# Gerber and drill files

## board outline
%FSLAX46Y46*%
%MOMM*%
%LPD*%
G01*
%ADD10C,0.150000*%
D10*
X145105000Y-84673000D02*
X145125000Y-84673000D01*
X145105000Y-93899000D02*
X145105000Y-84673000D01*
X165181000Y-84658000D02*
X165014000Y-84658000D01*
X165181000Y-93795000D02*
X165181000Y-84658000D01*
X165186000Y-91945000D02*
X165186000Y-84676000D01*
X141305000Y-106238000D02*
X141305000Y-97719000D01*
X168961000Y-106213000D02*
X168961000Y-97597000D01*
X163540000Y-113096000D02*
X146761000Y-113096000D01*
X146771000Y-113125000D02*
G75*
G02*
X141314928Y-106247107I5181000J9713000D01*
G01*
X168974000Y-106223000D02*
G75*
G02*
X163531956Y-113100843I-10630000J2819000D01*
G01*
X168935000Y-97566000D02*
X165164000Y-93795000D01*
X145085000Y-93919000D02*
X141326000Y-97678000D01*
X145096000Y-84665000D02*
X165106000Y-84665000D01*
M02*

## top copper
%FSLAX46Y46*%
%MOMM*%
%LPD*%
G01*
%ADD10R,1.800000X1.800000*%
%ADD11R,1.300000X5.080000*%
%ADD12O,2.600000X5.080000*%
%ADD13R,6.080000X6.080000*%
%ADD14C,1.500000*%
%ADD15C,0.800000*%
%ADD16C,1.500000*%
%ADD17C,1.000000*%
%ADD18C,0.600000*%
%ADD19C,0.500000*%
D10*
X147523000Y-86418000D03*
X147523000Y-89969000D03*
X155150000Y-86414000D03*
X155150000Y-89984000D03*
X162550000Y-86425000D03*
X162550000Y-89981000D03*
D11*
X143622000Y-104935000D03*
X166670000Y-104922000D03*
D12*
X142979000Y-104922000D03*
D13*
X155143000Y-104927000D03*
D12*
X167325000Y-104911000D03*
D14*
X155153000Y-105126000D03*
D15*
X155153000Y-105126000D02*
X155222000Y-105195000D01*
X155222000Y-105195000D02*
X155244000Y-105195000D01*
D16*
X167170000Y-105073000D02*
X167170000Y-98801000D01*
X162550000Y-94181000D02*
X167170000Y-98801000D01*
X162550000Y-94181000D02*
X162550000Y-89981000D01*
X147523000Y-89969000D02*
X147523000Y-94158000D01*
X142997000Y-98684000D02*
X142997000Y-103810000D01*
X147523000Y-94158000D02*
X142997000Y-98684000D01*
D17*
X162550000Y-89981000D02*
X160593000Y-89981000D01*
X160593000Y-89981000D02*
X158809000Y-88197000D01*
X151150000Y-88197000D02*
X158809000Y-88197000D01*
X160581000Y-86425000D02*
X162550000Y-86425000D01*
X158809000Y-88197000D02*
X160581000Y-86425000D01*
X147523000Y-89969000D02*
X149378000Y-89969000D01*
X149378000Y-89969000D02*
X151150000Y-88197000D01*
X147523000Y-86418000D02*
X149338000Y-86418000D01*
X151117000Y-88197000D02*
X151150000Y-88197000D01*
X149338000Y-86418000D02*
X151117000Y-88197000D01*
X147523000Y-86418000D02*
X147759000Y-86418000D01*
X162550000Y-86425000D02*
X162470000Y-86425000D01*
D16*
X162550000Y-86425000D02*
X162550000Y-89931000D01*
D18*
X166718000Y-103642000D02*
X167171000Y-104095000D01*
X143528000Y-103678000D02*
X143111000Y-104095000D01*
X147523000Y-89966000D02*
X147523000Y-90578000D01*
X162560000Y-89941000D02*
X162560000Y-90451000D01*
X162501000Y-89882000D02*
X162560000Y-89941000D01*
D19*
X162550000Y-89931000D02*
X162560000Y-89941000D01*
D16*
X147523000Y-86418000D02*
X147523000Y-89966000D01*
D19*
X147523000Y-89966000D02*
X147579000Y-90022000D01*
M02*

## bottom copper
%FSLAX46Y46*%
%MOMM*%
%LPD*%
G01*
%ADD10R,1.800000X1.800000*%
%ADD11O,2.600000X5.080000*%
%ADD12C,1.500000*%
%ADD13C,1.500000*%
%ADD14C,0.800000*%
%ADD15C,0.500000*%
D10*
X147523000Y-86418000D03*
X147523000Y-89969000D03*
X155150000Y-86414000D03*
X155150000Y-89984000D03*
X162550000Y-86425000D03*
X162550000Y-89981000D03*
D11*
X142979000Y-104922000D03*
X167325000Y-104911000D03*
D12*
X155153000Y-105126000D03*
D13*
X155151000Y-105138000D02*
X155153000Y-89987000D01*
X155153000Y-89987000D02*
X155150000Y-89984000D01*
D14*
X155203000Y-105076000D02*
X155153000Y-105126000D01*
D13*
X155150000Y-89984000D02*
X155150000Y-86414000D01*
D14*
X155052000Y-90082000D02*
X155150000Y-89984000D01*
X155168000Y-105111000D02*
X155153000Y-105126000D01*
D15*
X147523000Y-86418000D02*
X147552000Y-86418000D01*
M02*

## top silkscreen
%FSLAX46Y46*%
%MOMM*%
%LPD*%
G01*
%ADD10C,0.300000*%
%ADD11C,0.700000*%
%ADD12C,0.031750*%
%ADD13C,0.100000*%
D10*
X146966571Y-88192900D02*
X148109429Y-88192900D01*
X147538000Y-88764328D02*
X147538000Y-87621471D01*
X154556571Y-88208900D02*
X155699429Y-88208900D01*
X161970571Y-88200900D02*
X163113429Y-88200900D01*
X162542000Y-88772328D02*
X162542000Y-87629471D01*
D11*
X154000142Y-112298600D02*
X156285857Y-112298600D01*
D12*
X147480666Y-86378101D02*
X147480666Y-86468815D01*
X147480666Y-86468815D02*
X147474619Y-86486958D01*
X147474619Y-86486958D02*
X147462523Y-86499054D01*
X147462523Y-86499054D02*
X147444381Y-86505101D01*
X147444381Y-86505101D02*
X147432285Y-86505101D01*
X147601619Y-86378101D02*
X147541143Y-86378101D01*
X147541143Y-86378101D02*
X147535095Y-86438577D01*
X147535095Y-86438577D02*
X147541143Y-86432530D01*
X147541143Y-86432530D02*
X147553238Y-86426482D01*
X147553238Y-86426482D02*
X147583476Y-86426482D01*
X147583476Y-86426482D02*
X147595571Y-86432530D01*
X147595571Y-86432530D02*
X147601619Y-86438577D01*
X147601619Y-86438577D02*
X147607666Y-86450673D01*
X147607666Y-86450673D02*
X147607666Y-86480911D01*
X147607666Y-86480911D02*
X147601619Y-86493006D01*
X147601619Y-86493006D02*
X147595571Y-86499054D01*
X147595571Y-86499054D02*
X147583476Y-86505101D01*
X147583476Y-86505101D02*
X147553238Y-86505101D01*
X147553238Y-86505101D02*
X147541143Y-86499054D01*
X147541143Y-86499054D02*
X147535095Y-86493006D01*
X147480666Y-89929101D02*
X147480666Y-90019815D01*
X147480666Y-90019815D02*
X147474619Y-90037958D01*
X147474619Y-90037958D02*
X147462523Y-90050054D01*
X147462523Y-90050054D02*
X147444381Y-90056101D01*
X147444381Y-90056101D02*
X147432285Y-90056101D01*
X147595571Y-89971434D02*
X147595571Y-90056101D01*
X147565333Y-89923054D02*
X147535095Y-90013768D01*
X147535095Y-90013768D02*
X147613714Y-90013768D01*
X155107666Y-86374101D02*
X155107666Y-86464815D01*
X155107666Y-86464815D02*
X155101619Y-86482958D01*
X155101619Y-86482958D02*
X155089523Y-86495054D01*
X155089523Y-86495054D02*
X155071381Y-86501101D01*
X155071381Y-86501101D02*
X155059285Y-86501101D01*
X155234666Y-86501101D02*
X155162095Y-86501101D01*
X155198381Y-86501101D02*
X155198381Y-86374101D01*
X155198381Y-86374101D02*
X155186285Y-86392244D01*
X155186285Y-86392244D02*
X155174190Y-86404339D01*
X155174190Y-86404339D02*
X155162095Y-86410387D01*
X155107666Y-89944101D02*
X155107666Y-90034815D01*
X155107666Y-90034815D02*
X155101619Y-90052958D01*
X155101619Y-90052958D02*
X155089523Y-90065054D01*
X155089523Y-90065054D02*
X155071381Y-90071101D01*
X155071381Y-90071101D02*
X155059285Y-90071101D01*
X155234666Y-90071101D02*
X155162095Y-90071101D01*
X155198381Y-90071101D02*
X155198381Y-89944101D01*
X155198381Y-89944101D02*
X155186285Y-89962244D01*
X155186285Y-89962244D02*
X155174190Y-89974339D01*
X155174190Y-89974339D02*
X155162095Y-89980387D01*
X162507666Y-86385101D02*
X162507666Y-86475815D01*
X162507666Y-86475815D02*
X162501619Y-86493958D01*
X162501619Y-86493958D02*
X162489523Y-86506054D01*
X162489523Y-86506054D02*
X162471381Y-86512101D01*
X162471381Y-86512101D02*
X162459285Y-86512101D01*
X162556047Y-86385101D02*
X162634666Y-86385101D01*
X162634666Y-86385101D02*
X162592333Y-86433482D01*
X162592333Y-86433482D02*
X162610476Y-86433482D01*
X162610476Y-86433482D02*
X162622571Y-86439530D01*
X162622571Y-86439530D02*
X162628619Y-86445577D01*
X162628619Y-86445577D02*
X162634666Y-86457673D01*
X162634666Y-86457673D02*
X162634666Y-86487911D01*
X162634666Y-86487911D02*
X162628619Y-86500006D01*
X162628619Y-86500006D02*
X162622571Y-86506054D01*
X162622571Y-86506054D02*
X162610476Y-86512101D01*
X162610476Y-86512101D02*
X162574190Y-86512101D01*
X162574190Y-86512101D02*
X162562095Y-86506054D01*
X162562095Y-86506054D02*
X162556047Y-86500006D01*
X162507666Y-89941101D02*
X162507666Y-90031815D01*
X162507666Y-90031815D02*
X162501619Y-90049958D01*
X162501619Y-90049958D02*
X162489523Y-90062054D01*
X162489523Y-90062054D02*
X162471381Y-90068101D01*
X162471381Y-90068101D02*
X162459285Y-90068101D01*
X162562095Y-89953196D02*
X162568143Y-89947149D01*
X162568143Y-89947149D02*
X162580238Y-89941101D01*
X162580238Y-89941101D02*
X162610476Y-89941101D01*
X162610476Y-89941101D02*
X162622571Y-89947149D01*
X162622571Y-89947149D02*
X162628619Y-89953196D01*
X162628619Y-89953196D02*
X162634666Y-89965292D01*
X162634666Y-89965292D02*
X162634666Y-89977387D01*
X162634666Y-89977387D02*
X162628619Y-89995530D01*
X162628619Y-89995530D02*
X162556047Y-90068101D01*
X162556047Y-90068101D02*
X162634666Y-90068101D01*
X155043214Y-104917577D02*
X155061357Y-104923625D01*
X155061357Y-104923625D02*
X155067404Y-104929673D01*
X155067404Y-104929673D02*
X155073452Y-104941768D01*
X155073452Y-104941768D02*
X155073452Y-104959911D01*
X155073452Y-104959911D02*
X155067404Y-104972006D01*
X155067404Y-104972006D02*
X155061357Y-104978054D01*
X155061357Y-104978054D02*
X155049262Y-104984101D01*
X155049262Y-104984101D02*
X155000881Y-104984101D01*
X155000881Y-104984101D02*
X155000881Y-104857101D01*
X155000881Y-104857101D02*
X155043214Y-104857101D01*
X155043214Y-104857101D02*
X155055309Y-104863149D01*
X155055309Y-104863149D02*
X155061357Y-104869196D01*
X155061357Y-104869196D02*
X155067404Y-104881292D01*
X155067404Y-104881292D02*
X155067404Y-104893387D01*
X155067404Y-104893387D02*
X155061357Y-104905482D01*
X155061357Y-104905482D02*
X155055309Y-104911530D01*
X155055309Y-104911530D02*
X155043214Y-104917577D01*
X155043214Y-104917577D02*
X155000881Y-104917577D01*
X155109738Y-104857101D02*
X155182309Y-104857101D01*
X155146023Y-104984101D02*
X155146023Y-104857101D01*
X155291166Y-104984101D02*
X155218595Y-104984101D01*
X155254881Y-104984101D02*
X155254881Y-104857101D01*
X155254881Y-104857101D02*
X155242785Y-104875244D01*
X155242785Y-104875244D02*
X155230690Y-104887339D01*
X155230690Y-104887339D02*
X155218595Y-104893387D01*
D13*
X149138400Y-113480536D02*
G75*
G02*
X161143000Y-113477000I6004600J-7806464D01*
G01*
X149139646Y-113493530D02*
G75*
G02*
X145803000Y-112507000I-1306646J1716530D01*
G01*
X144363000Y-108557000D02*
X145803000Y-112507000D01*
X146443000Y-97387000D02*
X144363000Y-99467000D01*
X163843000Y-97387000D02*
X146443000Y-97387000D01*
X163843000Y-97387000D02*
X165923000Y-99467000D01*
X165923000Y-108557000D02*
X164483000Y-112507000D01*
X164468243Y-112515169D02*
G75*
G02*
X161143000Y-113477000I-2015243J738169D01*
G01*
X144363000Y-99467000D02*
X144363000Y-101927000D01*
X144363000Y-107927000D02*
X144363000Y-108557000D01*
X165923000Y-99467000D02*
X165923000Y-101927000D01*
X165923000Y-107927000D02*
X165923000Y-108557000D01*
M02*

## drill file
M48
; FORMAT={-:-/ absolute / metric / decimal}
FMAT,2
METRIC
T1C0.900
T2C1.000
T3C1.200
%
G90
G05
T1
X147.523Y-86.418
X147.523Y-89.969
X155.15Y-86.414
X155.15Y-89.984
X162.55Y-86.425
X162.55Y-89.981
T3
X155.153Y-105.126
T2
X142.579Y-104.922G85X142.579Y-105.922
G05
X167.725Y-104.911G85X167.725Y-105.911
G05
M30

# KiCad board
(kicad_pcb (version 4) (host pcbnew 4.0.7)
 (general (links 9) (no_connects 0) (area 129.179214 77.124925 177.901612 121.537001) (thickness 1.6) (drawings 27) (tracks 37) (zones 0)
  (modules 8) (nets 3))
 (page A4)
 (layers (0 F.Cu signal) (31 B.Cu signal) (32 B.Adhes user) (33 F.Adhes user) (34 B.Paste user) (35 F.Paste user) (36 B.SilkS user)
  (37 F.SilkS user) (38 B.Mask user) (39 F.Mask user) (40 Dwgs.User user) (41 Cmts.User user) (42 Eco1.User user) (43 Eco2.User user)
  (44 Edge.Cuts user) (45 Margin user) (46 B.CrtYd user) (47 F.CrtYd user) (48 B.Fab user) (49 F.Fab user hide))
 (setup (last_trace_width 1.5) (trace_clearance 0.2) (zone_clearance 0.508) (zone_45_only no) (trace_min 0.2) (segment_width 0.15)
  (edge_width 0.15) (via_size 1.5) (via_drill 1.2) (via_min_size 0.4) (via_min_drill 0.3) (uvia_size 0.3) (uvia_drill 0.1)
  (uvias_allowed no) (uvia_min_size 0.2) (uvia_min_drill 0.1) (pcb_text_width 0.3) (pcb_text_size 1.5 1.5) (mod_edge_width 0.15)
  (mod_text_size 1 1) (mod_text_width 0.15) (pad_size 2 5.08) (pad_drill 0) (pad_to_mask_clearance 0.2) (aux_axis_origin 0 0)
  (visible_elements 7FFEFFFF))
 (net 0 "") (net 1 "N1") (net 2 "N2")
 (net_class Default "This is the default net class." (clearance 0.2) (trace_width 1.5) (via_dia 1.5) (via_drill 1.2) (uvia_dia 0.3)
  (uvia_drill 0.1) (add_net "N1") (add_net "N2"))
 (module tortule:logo (layer B.Cu) (at 153.53 108.407)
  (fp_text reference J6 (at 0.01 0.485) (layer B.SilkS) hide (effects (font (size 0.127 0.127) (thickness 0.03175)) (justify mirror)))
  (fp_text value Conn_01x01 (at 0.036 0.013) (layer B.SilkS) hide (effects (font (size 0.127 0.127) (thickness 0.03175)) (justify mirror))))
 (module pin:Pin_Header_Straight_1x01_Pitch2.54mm (layer F.Cu) (at 147.523 86.418)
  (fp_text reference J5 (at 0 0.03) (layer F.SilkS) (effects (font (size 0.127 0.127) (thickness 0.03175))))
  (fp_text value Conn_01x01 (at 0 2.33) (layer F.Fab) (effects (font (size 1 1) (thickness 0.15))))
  (pad 1 thru_hole rect (at 0 0) (size 1.8 1.8) (drill 0.9) (layers *.Cu *.Mask) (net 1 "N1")))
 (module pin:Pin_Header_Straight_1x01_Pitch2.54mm (layer F.Cu) (at 147.523 89.969)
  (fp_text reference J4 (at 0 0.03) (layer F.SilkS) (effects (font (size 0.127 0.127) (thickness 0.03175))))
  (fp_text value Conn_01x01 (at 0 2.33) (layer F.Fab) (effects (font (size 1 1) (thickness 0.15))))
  (pad 1 thru_hole rect (at 0 0) (size 1.8 1.8) (drill 0.9) (layers *.Cu *.Mask) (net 1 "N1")))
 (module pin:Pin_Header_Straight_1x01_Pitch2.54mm (layer F.Cu) (at 155.15 86.414)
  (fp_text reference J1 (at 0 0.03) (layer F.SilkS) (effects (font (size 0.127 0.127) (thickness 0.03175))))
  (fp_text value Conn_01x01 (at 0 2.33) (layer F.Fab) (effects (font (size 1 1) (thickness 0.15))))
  (pad 1 thru_hole rect (at 0 0) (size 1.8 1.8) (drill 0.9) (layers *.Cu *.Mask) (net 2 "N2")))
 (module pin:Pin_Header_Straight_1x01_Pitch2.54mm (layer F.Cu) (at 155.15 89.984)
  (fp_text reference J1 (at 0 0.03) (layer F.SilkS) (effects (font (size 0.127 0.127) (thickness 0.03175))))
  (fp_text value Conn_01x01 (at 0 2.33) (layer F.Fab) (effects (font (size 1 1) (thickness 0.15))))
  (pad 1 thru_hole rect (at 0 0) (size 1.8 1.8) (drill 0.9) (layers *.Cu *.Mask) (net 2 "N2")))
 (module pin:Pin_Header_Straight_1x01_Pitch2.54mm (layer F.Cu) (at 162.55 86.425)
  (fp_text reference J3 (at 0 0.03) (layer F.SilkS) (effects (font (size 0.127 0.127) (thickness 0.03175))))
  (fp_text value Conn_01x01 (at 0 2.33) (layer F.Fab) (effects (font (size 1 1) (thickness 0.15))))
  (pad 1 thru_hole rect (at 0 0) (size 1.8 1.8) (drill 0.9) (layers *.Cu *.Mask) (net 1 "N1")))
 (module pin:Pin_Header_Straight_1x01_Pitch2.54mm (layer F.Cu) (at 162.55 89.981)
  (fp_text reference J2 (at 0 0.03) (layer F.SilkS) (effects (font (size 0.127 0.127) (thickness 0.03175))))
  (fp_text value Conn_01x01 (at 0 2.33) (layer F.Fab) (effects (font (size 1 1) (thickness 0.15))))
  (pad 1 thru_hole rect (at 0 0) (size 1.8 1.8) (drill 0.9) (layers *.Cu *.Mask) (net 1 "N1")))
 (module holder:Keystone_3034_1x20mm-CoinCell (layer F.Cu) (at 155.143 104.927)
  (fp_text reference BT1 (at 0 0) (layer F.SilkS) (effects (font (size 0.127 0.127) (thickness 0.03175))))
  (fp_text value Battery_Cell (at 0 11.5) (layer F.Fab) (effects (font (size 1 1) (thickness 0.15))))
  (fp_arc (start 0 16.36) (end 6 8.55) (angle -75.1) (layer F.SilkS) (width 0.1))
  (fp_arc (start -7.31 6.85) (end -9.34 7.58) (angle -107.5) (layer F.SilkS) (width 0.1))
  (fp_line (start -10.78 3.63) (end -9.34 7.58) (layer F.SilkS) (width 0.1))
  (fp_line (start -8.7 -7.54) (end -10.78 -5.46) (layer F.SilkS) (width 0.1))
  (fp_line (start 8.7 -7.54) (end -8.7 -7.54) (layer F.SilkS) (width 0.1))
  (fp_line (start 8.7 -7.54) (end 10.78 -5.46) (layer F.SilkS) (width 0.1))
  (fp_line (start 10.78 3.63) (end 9.34 7.58) (layer F.SilkS) (width 0.1))
  (fp_arc (start 7.31 6.85) (end 6 8.55) (angle -107.5) (layer F.SilkS) (width 0.1))
  (fp_line (start -10.78 -5.46) (end -10.78 -3) (layer F.SilkS) (width 0.1))
  (fp_line (start -10.78 3) (end -10.78 3.63) (layer F.SilkS) (width 0.1))
  (fp_line (start 10.78 -5.46) (end 10.78 -3) (layer F.SilkS) (width 0.1))
  (fp_line (start 10.78 3) (end 10.78 3.63) (layer F.SilkS) (width 0.1))
  (pad 1 smd rect (at -11.021 0.008) (size 1.3 5.08) (drill oval (offset -0.5 0)) (layers F.Cu F.Paste F.Mask) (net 1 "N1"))
  (pad 1 smd rect (at 12.027 -0.005) (size 1.3 5.08) (drill oval (offset -0.5 0)) (layers F.Cu F.Paste F.Mask) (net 1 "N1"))
  (pad 1 thru_hole oval (at -12.564 0.495) (size 2.6 5.08) (drill oval 1 2 (offset 0.4 -0.5)) (layers *.Cu *.Mask) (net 1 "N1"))
  (pad 2 smd rect (at 0 0) (size 6.08 6.08) (layers F.Cu F.Paste F.Mask) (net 2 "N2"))
  (pad 1 thru_hole oval (at 12.582 0.484) (size 2.6 5.08) (drill oval 1 2 (offset -0.4 -0.5)) (layers *.Cu *.Mask) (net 1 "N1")))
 (gr_line (start 145.105 84.673) (end 145.125 84.673) (angle 90) (layer Edge.Cuts) (width 0.15))
 (gr_line (start 145.105 93.899) (end 145.105 84.673) (angle 90) (layer Edge.Cuts) (width 0.15))
 (gr_line (start 165.181 84.658) (end 165.014 84.658) (angle 90) (layer Edge.Cuts) (width 0.15))
 (gr_line (start 165.181 93.795) (end 165.181 84.658) (angle 90) (layer Edge.Cuts) (width 0.15))
 (gr_line (start 165.186 91.945) (end 165.186 84.676) (angle 90) (layer Edge.Cuts) (width 0.15))
 (gr_line (start 141.305 106.238) (end 141.305 97.719) (angle 90) (layer Edge.Cuts) (width 0.15))
 (gr_line (start 168.961 106.213) (end 168.961 97.597) (angle 90) (layer Edge.Cuts) (width 0.15))
 (gr_line (start 163.54 113.096) (end 146.761 113.096) (angle 90) (layer Edge.Cuts) (width 0.15))
 (gr_arc (start 151.952 103.412) (end 146.771 113.125) (angle 47) (layer Edge.Cuts) (width 0.15))
 (gr_arc (start 158.344 103.404) (end 168.974 106.223) (angle 47) (layer Edge.Cuts) (width 0.15))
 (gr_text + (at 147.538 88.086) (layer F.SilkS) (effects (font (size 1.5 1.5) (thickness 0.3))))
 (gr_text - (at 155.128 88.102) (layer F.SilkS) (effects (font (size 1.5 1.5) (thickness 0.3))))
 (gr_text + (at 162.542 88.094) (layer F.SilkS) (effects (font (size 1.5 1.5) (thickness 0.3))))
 (gr_line (start 168.935 97.566) (end 165.164 93.795) (angle 90) (layer Edge.Cuts) (width 0.15))
 (gr_line (start 145.085 93.919) (end 141.326 97.678) (angle 90) (layer Edge.Cuts) (width 0.15))
 (gr_line (start 145.096 84.665) (end 165.106 84.665) (angle 90) (layer Edge.Cuts) (width 0.15))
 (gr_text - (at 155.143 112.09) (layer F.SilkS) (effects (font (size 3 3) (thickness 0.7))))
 (segment (start 155.151 105.138) (end 155.153 89.987) (width 1.5) (layer B.Cu) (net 2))
 (segment (start 155.153 89.987) (end 155.15 89.984) (width 1.5) (layer B.Cu) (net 2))
 (segment (start 155.203 105.076) (end 155.153 105.126) (width 0.8) (layer B.Cu) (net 2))
 (segment (start 155.15 89.984) (end 155.15 86.414) (width 1.5) (layer B.Cu) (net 2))
 (segment (start 155.052 90.082) (end 155.15 89.984) (width 0.8) (layer B.Cu) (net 2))
 (segment (start 155.153 105.126) (end 155.222 105.195) (width 0.8) (layer F.Cu) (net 2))
 (via (at 155.153 105.126) (size 1.5) (drill 1.2) (layers F.Cu B.Cu) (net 2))
 (segment (start 155.168 105.111) (end 155.153 105.126) (width 0.8) (layer B.Cu) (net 2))
 (segment (start 155.222 105.195) (end 155.244 105.195) (width 0.8) (layer F.Cu) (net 2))
 (segment (start 167.17 105.073) (end 167.17 98.801) (width 1.5) (layer F.Cu) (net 1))
 (segment (start 162.55 94.181) (end 167.17 98.801) (width 1.5) (layer F.Cu) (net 1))
 (segment (start 162.55 94.181) (end 162.55 89.981) (width 1.5) (layer F.Cu) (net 1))
 (segment (start 147.523 89.969) (end 147.523 94.158) (width 1.5) (layer F.Cu) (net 1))
 (segment (start 142.997 98.684) (end 142.997 103.81) (width 1.5) (layer F.Cu) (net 1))
 (segment (start 147.523 94.158) (end 142.997 98.684) (width 1.5) (layer F.Cu) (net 1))
 (segment (start 162.55 89.981) (end 160.593 89.981) (width 1) (layer F.Cu) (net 1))
 (segment (start 160.593 89.981) (end 158.809 88.197) (width 1) (layer F.Cu) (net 1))
 (segment (start 151.15 88.197) (end 158.809 88.197) (width 1) (layer F.Cu) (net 1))
 (segment (start 160.581 86.425) (end 162.55 86.425) (width 1) (layer F.Cu) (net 1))
 (segment (start 158.809 88.197) (end 160.581 86.425) (width 1) (layer F.Cu) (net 1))
 (segment (start 147.523 89.969) (end 149.378 89.969) (width 1) (layer F.Cu) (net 1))
 (segment (start 149.378 89.969) (end 151.15 88.197) (width 1) (layer F.Cu) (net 1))
 (segment (start 147.523 86.418) (end 149.338 86.418) (width 1) (layer F.Cu) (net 1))
 (segment (start 151.117 88.197) (end 151.15 88.197) (width 1) (layer F.Cu) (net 1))
 (segment (start 149.338 86.418) (end 151.117 88.197) (width 1) (layer F.Cu) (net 1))
 (segment (start 147.523 86.418) (end 147.759 86.418) (width 1) (layer F.Cu) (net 1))
 (segment (start 162.55 86.425) (end 162.47 86.425) (width 1) (layer F.Cu) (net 1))
 (segment (start 162.55 86.425) (end 162.55 89.931) (width 1.5) (layer F.Cu) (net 1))
 (segment (start 166.718 103.642) (end 167.171 104.095) (width 0.6) (layer F.Cu) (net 1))
 (segment (start 143.528 103.678) (end 143.111 104.095) (width 0.6) (layer F.Cu) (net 1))
 (segment (start 147.523 89.966) (end 147.523 90.578) (width 0.6) (layer F.Cu) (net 1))
 (segment (start 162.56 89.941) (end 162.56 90.451) (width 0.6) (layer F.Cu) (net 1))
 (segment (start 162.501 89.882) (end 162.56 89.941) (width 0.6) (layer F.Cu) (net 1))
 (segment (start 147.523 86.418) (end 147.552 86.418) (width 0.5) (layer B.Cu) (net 1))
 (segment (start 162.55 89.931) (end 162.56 89.941) (width 0.5) (layer F.Cu) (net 1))
 (segment (start 147.523 86.418) (end 147.523 89.966) (width 1.5) (layer F.Cu) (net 1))
 (segment (start 147.523 89.966) (end 147.579 90.022) (width 0.5) (layer F.Cu) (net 1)))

